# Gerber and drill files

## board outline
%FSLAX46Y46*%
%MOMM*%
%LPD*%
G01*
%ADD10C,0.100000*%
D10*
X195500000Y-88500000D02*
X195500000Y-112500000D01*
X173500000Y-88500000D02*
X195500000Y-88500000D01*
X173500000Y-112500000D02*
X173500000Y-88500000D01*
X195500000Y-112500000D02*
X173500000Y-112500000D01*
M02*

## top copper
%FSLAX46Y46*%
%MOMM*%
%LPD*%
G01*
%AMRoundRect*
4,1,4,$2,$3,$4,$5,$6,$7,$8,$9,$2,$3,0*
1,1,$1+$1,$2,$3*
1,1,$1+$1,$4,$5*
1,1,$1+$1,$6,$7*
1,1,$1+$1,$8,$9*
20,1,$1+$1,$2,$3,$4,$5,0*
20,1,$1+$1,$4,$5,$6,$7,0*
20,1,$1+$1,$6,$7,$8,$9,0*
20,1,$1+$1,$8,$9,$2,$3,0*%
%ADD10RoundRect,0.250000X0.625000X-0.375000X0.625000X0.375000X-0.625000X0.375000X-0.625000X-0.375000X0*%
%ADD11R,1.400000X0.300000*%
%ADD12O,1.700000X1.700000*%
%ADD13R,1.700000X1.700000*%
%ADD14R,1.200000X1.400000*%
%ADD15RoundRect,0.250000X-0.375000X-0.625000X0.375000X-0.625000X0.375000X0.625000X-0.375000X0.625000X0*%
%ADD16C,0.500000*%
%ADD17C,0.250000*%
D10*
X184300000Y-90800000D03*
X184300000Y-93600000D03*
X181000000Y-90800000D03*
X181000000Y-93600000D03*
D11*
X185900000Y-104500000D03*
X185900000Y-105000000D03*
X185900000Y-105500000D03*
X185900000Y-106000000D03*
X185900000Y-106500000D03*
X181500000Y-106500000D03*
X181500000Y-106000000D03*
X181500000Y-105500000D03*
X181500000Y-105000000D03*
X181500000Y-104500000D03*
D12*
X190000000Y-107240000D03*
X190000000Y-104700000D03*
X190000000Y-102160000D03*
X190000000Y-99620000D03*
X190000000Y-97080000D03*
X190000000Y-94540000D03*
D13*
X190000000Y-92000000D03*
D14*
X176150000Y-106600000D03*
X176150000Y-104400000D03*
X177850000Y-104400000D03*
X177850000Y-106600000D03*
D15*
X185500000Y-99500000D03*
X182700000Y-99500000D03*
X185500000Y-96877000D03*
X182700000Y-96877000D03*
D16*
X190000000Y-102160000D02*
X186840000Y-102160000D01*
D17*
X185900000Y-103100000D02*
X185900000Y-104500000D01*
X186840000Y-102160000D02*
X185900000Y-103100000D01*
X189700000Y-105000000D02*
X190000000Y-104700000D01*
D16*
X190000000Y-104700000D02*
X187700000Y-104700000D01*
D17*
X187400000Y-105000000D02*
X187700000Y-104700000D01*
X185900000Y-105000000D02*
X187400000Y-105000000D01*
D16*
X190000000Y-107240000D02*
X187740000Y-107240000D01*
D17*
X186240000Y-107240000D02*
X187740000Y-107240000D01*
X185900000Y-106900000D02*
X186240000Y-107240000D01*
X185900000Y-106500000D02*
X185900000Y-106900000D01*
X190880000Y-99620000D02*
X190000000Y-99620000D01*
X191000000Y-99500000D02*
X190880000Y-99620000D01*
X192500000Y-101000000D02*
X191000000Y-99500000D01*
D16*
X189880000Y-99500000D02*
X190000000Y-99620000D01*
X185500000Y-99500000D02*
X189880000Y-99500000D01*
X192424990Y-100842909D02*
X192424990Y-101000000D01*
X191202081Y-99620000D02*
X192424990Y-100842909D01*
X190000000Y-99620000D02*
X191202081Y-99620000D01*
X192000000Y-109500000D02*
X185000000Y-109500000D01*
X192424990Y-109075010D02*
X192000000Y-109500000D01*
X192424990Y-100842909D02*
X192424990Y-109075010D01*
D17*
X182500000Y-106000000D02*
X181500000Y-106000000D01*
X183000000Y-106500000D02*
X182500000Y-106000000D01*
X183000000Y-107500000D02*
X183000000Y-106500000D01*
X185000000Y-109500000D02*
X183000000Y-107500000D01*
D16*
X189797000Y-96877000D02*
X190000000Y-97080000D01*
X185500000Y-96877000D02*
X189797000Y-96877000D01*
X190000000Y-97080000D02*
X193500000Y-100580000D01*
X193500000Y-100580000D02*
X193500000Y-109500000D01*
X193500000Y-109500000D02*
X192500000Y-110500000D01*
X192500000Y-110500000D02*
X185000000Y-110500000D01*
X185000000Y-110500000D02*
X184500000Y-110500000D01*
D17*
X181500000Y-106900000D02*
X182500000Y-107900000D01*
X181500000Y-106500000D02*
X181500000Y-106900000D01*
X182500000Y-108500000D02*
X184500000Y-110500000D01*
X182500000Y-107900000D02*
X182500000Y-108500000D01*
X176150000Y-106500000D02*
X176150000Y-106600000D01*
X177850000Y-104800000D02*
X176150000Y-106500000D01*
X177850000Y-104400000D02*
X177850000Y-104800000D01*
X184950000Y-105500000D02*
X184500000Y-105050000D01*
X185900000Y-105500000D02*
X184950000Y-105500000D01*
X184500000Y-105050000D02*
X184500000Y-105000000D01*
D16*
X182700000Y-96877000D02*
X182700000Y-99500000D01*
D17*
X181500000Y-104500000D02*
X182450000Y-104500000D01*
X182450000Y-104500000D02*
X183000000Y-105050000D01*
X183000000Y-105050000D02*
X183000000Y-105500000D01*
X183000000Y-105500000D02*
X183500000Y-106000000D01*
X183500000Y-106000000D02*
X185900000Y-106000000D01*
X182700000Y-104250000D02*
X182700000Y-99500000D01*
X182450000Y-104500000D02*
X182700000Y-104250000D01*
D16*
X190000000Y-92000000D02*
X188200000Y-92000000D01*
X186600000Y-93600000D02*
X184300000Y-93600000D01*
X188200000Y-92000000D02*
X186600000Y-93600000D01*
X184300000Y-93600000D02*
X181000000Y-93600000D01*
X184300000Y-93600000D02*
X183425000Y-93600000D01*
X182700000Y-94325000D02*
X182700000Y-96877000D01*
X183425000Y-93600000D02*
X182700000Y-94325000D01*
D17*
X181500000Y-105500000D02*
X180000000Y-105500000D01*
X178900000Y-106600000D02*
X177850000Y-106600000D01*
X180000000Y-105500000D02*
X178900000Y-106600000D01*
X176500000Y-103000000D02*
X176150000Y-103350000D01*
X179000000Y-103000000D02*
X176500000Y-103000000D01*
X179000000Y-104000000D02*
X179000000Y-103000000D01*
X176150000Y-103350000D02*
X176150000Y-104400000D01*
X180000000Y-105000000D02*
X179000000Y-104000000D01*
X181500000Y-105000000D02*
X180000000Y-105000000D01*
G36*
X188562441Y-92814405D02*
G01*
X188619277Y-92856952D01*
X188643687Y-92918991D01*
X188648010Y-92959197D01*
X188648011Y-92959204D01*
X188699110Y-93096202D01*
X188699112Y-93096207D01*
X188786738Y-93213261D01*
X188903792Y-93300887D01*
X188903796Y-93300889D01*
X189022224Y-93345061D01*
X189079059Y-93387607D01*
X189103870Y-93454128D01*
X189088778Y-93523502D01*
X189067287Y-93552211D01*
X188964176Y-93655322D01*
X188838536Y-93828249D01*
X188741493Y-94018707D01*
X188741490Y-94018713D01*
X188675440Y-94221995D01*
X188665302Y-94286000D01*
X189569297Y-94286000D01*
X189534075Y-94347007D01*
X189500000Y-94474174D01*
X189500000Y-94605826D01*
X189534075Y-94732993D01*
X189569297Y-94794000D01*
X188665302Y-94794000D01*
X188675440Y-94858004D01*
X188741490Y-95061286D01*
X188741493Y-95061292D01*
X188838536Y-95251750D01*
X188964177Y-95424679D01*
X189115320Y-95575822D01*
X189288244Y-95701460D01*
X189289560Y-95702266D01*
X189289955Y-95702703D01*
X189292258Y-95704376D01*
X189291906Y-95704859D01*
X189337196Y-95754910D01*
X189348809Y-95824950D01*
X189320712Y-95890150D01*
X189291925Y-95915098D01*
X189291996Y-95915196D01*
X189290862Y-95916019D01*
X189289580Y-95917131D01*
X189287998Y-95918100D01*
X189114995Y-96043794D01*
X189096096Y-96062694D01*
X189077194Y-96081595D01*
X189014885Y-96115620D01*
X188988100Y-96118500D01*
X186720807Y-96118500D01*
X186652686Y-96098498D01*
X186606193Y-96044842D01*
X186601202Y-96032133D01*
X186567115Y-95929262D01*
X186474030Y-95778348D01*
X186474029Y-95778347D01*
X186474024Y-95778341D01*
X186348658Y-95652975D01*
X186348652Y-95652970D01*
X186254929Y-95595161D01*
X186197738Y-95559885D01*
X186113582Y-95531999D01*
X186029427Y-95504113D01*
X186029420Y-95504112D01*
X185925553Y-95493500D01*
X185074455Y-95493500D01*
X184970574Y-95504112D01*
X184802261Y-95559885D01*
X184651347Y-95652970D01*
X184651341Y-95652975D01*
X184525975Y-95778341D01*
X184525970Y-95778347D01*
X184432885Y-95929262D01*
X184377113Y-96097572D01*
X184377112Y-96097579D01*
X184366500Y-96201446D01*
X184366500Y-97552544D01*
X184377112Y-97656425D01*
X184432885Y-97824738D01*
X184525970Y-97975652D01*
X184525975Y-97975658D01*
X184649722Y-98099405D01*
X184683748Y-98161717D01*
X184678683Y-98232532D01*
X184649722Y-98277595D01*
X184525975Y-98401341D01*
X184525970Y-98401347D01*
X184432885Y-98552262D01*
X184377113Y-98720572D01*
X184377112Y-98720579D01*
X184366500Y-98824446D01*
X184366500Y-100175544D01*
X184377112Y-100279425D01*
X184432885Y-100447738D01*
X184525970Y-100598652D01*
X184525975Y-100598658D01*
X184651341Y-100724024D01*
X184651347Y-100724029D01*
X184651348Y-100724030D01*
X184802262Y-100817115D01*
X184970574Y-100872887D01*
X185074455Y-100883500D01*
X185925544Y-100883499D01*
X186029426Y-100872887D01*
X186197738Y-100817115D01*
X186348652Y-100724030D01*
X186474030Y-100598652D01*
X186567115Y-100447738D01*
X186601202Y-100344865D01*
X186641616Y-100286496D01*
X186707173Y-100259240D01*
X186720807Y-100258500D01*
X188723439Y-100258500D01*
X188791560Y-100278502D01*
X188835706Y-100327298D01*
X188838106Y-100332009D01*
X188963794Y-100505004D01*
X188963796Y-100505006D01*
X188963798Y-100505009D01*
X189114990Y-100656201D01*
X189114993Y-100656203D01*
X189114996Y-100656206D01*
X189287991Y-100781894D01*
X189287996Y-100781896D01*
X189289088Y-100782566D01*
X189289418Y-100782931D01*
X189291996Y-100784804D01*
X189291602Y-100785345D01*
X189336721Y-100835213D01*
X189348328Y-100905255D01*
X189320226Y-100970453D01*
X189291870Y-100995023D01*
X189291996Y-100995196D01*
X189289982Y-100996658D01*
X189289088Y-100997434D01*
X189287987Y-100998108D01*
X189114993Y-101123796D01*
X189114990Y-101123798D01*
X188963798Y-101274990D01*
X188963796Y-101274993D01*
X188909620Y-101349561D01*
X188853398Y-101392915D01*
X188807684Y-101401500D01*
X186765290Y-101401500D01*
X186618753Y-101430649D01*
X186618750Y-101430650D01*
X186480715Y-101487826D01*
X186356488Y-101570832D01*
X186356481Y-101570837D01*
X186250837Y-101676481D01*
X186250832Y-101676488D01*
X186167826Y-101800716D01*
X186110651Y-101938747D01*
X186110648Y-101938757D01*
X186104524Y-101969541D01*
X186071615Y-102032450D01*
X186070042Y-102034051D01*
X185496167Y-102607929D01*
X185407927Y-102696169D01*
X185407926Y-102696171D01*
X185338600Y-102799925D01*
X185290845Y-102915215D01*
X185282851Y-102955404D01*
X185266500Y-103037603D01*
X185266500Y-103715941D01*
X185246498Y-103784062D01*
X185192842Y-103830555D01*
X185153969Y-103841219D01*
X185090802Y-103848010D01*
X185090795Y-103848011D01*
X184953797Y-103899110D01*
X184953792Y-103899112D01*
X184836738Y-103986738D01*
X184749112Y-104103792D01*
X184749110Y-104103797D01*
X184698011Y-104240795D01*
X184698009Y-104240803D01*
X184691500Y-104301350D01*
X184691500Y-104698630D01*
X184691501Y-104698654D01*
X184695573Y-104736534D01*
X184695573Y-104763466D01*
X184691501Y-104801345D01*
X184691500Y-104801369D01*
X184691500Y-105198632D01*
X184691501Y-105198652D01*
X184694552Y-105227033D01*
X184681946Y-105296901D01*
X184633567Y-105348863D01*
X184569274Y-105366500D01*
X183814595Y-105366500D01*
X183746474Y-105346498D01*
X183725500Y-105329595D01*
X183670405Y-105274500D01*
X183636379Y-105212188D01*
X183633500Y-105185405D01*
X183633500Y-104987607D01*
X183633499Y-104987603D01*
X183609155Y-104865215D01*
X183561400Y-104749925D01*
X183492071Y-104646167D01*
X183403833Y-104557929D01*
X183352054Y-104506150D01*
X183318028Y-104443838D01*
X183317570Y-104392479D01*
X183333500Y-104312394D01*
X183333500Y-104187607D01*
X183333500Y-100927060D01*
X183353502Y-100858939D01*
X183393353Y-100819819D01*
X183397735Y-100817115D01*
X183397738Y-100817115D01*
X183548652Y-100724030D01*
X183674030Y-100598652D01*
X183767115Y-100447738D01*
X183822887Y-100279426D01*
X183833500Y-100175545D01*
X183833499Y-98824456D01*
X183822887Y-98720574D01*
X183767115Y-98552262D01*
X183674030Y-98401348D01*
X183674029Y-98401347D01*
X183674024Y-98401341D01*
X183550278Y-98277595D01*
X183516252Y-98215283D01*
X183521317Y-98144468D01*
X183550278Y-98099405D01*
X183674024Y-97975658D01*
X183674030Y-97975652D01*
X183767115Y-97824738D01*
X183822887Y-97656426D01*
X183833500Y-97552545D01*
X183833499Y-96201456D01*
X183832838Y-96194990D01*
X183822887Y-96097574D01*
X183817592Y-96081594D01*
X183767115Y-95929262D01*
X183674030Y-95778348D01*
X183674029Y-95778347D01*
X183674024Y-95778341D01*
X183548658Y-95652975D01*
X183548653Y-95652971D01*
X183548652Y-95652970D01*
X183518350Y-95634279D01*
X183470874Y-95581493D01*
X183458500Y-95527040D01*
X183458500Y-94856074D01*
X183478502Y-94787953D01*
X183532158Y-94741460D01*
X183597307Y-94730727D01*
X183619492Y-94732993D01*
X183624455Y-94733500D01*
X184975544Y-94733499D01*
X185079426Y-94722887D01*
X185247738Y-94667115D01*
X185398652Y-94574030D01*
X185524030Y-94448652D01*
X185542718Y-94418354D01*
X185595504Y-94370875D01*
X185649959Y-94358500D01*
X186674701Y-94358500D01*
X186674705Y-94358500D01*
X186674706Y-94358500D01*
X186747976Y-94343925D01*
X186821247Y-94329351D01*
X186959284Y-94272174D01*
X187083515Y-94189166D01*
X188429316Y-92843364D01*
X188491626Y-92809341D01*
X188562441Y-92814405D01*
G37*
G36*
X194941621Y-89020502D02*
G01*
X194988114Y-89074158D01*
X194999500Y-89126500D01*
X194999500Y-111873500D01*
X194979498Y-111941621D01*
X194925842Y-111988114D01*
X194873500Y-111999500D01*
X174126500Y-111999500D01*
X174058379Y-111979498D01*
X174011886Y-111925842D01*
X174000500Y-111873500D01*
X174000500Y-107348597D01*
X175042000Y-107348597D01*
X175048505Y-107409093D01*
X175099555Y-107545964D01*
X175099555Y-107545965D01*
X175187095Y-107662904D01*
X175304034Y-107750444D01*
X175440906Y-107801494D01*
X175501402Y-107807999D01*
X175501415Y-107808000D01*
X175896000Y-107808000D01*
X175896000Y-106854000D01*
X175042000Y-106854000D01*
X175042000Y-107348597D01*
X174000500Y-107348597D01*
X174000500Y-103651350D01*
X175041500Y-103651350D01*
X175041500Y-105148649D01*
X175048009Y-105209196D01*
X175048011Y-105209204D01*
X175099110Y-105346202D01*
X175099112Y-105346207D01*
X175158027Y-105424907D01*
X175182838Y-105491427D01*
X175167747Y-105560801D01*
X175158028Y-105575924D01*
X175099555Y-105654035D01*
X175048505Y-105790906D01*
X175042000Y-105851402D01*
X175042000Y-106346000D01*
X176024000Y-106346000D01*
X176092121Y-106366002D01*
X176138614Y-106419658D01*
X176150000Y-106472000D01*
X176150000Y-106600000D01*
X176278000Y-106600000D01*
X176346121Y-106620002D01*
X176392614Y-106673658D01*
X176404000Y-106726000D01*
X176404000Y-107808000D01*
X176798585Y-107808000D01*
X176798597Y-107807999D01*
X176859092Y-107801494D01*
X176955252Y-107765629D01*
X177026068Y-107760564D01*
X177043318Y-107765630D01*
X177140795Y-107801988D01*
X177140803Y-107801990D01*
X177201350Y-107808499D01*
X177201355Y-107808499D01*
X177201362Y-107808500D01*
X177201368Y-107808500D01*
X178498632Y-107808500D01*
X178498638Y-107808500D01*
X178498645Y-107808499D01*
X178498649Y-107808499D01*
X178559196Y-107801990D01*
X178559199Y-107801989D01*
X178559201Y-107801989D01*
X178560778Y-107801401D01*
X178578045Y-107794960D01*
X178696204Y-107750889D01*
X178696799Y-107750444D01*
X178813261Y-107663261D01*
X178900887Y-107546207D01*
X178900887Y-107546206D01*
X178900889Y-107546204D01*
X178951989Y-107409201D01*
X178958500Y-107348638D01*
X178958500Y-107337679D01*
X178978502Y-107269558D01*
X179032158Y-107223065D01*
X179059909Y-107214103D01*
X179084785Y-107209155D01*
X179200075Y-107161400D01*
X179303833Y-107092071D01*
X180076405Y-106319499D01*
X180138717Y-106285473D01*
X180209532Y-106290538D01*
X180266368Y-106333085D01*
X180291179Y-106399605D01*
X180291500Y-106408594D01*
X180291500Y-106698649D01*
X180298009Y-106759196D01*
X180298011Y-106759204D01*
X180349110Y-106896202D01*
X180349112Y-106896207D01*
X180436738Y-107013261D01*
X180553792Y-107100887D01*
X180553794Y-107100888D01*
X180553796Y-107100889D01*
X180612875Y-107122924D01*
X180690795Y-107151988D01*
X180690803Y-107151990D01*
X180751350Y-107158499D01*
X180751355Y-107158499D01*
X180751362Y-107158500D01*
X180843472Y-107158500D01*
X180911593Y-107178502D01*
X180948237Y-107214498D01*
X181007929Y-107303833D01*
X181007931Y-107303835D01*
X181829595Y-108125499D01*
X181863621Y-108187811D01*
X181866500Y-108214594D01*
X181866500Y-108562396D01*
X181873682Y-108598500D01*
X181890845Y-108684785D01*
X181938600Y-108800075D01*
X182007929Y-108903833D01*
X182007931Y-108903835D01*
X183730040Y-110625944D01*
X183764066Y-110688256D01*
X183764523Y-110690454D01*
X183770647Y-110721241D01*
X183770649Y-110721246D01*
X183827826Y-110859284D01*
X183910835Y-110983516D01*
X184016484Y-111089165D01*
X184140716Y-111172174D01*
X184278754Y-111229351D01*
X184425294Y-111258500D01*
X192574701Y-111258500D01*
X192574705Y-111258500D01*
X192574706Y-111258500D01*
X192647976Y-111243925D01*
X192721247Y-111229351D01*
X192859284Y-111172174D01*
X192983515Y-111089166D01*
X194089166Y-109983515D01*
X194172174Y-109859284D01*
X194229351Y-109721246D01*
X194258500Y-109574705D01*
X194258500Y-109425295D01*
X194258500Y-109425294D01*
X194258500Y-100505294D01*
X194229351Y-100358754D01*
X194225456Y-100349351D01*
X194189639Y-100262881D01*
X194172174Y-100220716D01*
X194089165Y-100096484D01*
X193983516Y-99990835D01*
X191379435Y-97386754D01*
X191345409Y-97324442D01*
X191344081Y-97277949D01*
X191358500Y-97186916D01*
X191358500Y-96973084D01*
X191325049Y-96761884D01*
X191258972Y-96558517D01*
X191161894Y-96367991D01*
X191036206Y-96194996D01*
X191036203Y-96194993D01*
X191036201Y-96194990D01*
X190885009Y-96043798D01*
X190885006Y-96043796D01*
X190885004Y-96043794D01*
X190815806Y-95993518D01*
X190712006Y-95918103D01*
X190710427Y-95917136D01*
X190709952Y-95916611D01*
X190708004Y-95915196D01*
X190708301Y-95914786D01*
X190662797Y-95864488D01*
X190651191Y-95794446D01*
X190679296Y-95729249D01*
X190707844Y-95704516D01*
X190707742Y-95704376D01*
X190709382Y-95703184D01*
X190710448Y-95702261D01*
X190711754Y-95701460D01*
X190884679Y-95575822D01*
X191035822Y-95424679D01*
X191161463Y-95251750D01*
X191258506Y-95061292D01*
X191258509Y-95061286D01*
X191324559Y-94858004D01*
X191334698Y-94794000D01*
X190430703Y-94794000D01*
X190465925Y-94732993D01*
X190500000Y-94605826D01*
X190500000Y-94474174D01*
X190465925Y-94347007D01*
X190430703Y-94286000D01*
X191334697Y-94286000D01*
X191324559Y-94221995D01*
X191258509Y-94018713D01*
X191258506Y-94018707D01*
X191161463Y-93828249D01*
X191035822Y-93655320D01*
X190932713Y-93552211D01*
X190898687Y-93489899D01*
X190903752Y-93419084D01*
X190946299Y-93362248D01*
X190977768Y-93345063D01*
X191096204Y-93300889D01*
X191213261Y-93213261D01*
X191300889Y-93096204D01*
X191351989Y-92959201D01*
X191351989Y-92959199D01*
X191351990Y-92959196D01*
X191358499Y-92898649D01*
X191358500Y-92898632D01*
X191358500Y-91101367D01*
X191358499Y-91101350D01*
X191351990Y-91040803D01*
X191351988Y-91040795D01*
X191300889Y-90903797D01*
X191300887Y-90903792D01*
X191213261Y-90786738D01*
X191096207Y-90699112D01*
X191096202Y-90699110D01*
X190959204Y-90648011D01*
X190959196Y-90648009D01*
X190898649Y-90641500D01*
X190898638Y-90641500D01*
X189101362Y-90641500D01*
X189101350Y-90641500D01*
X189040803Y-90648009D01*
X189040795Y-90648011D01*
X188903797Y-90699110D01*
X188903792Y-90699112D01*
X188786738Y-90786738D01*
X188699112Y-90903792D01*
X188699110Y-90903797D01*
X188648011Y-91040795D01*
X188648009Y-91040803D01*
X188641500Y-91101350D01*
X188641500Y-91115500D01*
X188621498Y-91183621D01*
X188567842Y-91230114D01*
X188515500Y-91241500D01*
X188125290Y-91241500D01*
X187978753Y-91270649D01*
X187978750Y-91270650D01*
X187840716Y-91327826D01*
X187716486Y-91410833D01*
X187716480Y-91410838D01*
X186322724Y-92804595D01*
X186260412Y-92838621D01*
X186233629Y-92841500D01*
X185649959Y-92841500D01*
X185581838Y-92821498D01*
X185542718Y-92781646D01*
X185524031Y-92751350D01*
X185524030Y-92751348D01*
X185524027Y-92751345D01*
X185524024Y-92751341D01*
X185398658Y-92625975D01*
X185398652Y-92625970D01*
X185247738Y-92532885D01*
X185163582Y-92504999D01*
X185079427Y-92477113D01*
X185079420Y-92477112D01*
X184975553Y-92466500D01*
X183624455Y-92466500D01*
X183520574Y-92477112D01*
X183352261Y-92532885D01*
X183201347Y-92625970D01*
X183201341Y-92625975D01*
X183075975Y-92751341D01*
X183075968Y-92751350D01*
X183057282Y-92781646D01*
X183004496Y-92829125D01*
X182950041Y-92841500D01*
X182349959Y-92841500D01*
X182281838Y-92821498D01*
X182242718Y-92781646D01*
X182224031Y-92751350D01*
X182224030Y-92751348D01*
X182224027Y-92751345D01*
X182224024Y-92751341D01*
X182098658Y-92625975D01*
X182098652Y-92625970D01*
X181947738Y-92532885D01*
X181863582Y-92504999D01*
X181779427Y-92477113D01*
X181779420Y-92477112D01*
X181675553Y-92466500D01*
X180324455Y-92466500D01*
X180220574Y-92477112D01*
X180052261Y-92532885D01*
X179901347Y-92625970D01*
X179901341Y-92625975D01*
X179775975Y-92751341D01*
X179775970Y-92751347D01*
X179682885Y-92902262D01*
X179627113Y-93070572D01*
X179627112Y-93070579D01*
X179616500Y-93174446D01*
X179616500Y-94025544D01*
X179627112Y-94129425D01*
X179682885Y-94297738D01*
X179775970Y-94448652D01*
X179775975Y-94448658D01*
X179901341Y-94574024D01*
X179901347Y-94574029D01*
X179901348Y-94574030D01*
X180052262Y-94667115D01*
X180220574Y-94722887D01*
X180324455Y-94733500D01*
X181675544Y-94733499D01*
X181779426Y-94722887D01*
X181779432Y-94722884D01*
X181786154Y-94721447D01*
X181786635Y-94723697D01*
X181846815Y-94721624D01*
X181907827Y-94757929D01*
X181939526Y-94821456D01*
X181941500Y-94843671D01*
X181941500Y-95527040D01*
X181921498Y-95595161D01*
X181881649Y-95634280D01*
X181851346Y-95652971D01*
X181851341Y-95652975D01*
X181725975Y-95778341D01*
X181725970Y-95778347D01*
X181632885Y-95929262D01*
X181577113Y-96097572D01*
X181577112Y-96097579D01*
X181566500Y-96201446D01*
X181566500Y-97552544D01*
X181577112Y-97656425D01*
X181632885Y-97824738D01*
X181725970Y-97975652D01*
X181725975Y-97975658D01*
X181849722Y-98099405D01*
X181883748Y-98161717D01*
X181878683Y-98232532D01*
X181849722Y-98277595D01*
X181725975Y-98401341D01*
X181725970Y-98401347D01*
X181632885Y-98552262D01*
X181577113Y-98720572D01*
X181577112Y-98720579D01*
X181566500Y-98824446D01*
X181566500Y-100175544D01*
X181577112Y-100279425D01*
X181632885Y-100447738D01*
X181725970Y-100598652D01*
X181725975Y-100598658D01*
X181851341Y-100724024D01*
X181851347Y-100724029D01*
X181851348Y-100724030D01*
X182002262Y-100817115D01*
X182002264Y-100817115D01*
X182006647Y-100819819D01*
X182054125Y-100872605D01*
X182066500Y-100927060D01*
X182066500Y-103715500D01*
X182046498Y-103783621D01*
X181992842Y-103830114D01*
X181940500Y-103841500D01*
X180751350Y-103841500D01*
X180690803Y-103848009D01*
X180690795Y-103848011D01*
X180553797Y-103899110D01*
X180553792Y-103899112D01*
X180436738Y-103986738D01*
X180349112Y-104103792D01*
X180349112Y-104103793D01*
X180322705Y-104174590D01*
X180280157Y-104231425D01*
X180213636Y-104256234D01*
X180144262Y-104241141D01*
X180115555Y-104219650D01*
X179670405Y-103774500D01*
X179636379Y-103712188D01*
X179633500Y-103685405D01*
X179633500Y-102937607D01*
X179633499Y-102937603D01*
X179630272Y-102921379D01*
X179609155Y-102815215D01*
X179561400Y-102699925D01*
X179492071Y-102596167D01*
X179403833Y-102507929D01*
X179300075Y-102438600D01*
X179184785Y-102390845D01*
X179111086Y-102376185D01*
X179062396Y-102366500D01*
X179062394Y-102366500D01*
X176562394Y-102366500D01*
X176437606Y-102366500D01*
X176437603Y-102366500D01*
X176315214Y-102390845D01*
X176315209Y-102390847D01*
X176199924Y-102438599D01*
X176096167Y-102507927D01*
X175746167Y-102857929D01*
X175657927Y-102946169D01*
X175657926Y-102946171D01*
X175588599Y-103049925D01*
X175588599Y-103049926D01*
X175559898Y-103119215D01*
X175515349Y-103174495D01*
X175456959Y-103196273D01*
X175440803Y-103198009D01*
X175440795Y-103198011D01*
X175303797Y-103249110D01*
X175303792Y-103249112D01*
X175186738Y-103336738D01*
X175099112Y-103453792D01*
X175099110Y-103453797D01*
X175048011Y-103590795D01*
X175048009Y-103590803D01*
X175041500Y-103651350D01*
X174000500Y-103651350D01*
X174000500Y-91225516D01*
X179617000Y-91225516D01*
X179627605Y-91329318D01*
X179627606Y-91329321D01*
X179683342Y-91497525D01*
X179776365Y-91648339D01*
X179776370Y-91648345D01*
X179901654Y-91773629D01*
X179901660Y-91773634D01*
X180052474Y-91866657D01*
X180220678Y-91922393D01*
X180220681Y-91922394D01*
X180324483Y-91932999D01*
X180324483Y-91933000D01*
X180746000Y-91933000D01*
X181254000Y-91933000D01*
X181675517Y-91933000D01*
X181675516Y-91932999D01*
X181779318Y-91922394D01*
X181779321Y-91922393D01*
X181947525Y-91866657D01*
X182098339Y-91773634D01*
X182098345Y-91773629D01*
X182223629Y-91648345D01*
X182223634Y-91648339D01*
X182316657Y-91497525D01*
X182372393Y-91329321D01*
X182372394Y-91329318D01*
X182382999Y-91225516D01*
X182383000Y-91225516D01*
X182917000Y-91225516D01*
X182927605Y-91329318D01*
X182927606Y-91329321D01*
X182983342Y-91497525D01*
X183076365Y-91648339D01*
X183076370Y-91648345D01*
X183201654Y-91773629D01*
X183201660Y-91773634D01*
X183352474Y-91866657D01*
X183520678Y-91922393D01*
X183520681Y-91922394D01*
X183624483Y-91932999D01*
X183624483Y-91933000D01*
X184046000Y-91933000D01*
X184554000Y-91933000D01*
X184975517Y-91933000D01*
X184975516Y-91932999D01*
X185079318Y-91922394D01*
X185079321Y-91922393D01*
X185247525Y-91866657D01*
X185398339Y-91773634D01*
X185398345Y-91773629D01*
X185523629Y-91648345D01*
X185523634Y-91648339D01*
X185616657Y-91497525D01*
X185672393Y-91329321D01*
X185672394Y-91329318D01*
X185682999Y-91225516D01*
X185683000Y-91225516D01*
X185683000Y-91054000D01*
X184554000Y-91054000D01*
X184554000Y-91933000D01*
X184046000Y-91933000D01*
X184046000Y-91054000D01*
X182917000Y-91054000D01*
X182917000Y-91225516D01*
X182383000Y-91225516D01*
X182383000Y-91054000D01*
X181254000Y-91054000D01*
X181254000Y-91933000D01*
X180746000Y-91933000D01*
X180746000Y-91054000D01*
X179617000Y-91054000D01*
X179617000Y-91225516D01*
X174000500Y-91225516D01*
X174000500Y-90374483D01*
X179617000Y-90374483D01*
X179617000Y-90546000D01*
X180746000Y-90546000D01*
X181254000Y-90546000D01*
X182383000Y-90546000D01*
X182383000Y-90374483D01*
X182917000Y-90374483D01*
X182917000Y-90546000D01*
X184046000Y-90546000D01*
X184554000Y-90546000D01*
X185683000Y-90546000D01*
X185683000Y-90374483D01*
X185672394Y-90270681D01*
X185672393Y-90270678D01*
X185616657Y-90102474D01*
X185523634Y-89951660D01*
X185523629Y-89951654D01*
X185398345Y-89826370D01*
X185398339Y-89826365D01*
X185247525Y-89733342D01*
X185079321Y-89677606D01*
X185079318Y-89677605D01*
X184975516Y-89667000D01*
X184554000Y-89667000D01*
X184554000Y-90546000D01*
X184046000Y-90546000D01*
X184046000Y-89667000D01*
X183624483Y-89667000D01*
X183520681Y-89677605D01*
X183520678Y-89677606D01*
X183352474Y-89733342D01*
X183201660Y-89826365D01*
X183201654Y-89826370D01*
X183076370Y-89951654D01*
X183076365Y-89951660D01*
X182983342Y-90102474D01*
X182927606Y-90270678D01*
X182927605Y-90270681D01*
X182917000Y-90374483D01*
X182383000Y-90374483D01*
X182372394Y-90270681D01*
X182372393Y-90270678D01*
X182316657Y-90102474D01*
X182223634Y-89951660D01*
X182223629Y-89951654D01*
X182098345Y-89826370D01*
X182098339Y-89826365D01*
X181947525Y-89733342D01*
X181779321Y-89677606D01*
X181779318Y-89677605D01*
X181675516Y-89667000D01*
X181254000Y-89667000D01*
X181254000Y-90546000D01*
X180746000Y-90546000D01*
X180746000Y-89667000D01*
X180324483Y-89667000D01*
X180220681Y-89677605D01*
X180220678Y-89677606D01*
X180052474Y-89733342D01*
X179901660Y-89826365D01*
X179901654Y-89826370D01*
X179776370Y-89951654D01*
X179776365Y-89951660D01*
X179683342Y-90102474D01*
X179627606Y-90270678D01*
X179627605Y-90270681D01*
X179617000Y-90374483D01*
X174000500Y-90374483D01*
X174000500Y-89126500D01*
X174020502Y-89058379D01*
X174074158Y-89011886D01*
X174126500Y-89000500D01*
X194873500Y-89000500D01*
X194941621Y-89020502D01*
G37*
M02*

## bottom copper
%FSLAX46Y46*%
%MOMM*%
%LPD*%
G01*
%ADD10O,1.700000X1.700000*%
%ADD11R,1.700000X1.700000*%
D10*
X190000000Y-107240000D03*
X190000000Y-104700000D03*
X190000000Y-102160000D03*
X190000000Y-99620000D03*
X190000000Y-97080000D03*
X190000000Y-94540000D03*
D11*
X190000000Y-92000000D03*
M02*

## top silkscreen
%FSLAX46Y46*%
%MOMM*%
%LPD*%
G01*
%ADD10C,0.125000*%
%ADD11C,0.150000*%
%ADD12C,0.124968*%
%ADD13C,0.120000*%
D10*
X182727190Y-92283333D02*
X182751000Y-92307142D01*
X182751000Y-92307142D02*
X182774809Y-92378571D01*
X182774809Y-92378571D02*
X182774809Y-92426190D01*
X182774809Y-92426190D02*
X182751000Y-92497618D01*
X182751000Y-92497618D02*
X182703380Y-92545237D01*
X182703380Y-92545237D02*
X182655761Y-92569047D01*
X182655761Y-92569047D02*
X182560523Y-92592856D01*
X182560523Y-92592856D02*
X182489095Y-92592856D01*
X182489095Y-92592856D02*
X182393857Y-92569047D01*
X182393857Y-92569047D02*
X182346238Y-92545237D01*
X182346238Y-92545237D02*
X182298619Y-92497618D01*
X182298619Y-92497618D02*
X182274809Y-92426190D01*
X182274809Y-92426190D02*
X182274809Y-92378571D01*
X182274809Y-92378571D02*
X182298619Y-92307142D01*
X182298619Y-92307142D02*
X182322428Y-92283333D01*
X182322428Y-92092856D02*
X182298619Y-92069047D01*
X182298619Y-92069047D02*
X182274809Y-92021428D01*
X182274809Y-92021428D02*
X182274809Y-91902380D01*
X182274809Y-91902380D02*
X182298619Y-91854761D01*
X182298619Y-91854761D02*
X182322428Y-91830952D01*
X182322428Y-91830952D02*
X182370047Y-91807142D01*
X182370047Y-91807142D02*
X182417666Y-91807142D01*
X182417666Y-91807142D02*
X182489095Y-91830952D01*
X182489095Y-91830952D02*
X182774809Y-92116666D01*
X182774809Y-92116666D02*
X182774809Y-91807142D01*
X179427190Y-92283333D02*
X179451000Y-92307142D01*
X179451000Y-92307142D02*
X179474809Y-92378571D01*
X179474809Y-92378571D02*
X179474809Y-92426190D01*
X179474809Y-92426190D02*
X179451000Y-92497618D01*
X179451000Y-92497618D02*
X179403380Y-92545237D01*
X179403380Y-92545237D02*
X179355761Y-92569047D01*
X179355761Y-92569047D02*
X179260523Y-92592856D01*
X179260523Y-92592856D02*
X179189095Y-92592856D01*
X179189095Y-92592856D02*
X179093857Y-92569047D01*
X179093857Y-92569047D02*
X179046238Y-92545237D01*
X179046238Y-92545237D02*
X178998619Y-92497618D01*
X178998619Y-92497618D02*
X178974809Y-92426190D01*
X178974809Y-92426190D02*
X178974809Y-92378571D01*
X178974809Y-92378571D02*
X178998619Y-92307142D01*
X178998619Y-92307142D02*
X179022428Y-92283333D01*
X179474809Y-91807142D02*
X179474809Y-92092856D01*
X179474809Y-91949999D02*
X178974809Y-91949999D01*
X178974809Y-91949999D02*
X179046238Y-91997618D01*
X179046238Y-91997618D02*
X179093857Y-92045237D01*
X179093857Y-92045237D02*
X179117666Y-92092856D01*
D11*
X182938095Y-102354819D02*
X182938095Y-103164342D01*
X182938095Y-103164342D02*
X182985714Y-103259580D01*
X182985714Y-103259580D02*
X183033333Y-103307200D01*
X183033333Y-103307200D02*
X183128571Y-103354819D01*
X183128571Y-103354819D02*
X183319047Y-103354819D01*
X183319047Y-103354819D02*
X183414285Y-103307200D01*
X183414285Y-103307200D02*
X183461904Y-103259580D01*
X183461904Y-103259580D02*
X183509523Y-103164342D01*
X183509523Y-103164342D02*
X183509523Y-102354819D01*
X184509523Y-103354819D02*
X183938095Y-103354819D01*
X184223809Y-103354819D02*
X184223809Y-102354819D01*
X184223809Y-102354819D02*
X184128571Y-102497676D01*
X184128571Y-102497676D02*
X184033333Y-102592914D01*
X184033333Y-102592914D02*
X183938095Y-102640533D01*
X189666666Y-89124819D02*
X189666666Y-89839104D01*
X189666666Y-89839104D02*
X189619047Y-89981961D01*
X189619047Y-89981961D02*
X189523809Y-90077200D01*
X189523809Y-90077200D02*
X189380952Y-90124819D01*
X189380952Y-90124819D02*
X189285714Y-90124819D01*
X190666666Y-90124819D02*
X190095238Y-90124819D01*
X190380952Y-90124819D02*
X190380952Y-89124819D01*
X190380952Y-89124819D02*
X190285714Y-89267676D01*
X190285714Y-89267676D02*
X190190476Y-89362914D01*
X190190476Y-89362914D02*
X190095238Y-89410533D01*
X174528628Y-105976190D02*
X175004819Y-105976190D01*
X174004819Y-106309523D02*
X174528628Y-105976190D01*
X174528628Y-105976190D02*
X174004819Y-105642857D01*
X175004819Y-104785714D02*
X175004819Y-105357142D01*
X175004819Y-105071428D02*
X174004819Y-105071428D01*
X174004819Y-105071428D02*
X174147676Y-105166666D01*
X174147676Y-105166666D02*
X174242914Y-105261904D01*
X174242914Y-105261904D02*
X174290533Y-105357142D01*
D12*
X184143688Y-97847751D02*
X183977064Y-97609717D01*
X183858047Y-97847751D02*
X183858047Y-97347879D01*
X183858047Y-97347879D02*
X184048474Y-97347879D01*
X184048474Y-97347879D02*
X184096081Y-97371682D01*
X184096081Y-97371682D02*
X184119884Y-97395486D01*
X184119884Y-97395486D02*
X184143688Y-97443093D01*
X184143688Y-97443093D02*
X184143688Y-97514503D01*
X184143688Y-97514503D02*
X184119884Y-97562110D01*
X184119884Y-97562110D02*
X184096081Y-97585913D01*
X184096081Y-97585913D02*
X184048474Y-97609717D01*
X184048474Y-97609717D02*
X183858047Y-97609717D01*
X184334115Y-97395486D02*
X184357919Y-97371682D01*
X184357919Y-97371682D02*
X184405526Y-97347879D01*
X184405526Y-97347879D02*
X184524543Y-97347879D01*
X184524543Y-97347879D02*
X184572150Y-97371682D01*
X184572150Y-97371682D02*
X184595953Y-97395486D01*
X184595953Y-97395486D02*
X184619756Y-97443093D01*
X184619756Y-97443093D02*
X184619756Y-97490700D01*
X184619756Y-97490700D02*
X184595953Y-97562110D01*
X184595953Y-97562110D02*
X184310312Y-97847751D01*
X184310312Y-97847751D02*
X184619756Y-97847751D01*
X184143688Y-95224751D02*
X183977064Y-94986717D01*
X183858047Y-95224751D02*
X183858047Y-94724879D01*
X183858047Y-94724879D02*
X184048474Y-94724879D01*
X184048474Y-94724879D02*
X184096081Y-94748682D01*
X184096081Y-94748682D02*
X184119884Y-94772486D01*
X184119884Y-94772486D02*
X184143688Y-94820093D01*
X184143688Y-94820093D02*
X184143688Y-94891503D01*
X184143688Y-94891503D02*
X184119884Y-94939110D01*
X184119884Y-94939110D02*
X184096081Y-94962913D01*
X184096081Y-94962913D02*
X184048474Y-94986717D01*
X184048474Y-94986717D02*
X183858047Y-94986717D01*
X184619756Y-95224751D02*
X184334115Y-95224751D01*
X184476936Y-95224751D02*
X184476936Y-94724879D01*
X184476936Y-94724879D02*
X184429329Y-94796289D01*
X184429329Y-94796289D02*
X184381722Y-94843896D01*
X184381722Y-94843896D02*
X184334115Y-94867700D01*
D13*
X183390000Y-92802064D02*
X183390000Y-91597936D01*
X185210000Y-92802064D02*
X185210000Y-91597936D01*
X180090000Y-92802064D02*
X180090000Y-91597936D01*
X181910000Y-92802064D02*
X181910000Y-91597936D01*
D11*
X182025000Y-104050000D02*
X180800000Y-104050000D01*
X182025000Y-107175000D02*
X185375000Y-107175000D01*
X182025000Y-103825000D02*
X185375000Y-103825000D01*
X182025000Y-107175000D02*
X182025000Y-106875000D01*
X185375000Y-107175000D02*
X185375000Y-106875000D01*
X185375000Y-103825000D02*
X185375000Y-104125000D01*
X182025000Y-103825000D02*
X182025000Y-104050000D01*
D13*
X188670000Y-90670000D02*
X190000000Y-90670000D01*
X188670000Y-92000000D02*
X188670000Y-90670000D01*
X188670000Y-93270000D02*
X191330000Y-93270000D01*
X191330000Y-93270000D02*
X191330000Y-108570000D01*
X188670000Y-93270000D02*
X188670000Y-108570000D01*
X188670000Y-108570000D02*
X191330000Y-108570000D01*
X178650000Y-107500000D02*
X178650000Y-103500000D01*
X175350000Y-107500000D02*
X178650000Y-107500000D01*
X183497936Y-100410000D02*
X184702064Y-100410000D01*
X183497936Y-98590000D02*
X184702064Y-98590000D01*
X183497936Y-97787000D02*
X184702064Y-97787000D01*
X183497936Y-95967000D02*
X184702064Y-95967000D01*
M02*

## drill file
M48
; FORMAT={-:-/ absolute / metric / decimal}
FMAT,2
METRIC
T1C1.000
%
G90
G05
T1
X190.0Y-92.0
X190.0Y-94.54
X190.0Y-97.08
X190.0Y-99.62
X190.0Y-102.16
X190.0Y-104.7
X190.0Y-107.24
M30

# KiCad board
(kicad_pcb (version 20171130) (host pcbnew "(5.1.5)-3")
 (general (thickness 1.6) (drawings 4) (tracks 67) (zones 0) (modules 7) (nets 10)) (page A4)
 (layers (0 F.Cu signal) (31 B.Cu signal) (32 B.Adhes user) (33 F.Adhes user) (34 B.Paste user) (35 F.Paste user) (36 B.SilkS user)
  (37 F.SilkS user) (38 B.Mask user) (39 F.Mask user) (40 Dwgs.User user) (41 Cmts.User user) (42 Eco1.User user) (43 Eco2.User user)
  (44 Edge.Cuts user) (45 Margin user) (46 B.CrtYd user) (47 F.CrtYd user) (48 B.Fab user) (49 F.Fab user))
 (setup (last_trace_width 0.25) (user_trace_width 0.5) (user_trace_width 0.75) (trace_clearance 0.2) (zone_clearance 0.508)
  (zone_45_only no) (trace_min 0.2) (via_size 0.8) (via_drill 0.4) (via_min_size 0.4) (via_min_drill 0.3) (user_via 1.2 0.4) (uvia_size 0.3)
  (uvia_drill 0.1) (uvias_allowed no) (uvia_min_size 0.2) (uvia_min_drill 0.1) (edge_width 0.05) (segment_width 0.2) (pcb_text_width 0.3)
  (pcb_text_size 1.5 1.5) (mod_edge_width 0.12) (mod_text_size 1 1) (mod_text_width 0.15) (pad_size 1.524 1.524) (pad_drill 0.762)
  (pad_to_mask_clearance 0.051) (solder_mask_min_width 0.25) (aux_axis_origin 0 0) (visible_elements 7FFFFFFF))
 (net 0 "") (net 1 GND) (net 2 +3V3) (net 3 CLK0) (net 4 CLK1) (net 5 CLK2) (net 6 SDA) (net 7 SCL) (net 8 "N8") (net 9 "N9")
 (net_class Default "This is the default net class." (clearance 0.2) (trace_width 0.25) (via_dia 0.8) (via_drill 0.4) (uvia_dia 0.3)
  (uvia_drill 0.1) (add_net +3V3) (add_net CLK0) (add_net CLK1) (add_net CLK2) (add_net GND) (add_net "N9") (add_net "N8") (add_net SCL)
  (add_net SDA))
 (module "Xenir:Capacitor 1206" (layer F.Cu) (at 182.05 92.2 90)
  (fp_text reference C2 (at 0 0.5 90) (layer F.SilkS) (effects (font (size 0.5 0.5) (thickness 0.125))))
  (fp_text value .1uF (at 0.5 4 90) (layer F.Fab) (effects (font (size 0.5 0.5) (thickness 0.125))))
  (fp_line (start -0.602064 1.34) (end 0.602064 1.34) (layer F.SilkS) (width 0.12))
  (fp_line (start -0.602064 3.16) (end 0.602064 3.16) (layer F.SilkS) (width 0.12))
  (pad 2 smd roundrect (at 1.4 2.25 90) (size 1.25 1.75) (layers F.Cu F.Paste F.Mask) (roundrect_rratio 0.2) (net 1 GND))
  (pad 1 smd roundrect (at -1.4 2.25 90) (size 1.25 1.75) (layers F.Cu F.Paste F.Mask) (roundrect_rratio 0.2) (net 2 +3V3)))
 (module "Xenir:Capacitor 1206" (layer F.Cu) (at 178.75 92.2 90)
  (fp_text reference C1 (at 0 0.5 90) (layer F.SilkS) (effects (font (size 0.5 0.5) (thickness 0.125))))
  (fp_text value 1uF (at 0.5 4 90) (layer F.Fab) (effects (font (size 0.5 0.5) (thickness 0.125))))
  (fp_line (start -0.602064 1.34) (end 0.602064 1.34) (layer F.SilkS) (width 0.12))
  (fp_line (start -0.602064 3.16) (end 0.602064 3.16) (layer F.SilkS) (width 0.12))
  (pad 2 smd roundrect (at 1.4 2.25 90) (size 1.25 1.75) (layers F.Cu F.Paste F.Mask) (roundrect_rratio 0.2) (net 1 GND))
  (pad 1 smd roundrect (at -1.4 2.25 90) (size 1.25 1.75) (layers F.Cu F.Paste F.Mask) (roundrect_rratio 0.2) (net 2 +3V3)))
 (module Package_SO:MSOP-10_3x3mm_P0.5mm (layer F.Cu) (at 183.7 105.5)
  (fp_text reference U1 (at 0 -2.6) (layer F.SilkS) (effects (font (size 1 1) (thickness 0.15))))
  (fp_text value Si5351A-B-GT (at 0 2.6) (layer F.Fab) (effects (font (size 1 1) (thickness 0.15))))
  (fp_line (start -1.675 -1.45) (end -2.9 -1.45) (layer F.SilkS) (width 0.15))
  (fp_line (start -1.675 1.675) (end 1.675 1.675) (layer F.SilkS) (width 0.15))
  (fp_line (start -1.675 -1.675) (end 1.675 -1.675) (layer F.SilkS) (width 0.15))
  (fp_line (start -1.675 1.675) (end -1.675 1.375) (layer F.SilkS) (width 0.15))
  (fp_line (start 1.675 1.675) (end 1.675 1.375) (layer F.SilkS) (width 0.15))
  (fp_line (start 1.675 -1.675) (end 1.675 -1.375) (layer F.SilkS) (width 0.15))
  (fp_line (start -1.675 -1.675) (end -1.675 -1.45) (layer F.SilkS) (width 0.15))
  (pad 10 smd rect (at 2.2 -1) (size 1.4 0.3) (layers F.Cu F.Paste F.Mask) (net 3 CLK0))
  (pad 9 smd rect (at 2.2 -0.5) (size 1.4 0.3) (layers F.Cu F.Paste F.Mask) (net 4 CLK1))
  (pad 8 smd rect (at 2.2 0) (size 1.4 0.3) (layers F.Cu F.Paste F.Mask) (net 1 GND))
  (pad 7 smd rect (at 2.2 0.5) (size 1.4 0.3) (layers F.Cu F.Paste F.Mask) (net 2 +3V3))
  (pad 6 smd rect (at 2.2 1) (size 1.4 0.3) (layers F.Cu F.Paste F.Mask) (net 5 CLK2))
  (pad 5 smd rect (at -2.2 1) (size 1.4 0.3) (layers F.Cu F.Paste F.Mask) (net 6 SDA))
  (pad 4 smd rect (at -2.2 0.5) (size 1.4 0.3) (layers F.Cu F.Paste F.Mask) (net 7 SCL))
  (pad 3 smd rect (at -2.2 0) (size 1.4 0.3) (layers F.Cu F.Paste F.Mask) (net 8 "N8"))
  (pad 2 smd rect (at -2.2 -0.5) (size 1.4 0.3) (layers F.Cu F.Paste F.Mask) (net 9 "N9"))
  (pad 1 smd rect (at -2.2 -1) (size 1.4 0.3) (layers F.Cu F.Paste F.Mask) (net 2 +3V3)))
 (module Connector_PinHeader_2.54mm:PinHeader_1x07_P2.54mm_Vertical (layer F.Cu) (at 190 92)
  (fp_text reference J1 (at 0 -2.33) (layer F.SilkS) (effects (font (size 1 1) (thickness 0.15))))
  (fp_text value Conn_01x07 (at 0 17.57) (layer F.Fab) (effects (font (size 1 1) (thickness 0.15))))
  (fp_line (start -1.33 -1.33) (end 0 -1.33) (layer F.SilkS) (width 0.12))
  (fp_line (start -1.33 0) (end -1.33 -1.33) (layer F.SilkS) (width 0.12))
  (fp_line (start -1.33 1.27) (end 1.33 1.27) (layer F.SilkS) (width 0.12))
  (fp_line (start 1.33 1.27) (end 1.33 16.57) (layer F.SilkS) (width 0.12))
  (fp_line (start -1.33 1.27) (end -1.33 16.57) (layer F.SilkS) (width 0.12))
  (fp_line (start -1.33 16.57) (end 1.33 16.57) (layer F.SilkS) (width 0.12))
  (pad 7 thru_hole oval (at 0 15.24) (size 1.7 1.7) (drill 1) (layers *.Cu *.Mask) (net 5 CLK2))
  (pad 6 thru_hole oval (at 0 12.7) (size 1.7 1.7) (drill 1) (layers *.Cu *.Mask) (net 4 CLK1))
  (pad 5 thru_hole oval (at 0 10.16) (size 1.7 1.7) (drill 1) (layers *.Cu *.Mask) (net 3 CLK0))
  (pad 4 thru_hole oval (at 0 7.62) (size 1.7 1.7) (drill 1) (layers *.Cu *.Mask) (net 7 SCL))
  (pad 3 thru_hole oval (at 0 5.08) (size 1.7 1.7) (drill 1) (layers *.Cu *.Mask) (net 6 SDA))
  (pad 2 thru_hole oval (at 0 2.54) (size 1.7 1.7) (drill 1) (layers *.Cu *.Mask) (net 1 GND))
  (pad 1 thru_hole rect (at 0 0) (size 1.7 1.7) (drill 1) (layers *.Cu *.Mask) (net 2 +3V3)))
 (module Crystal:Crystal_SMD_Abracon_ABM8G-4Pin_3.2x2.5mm (layer F.Cu) (at 177 105.5 90)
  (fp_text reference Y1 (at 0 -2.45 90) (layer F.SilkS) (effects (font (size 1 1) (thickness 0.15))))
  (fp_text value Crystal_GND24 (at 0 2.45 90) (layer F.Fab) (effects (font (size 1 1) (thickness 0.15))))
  (fp_line (start -2 1.65) (end 2 1.65) (layer F.SilkS) (width 0.12))
  (fp_line (start -2 -1.65) (end -2 1.65) (layer F.SilkS) (width 0.12))
  (pad 4 smd rect (at -1.1 -0.85 90) (size 1.4 1.2) (layers F.Cu F.Paste F.Mask) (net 1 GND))
  (pad 3 smd rect (at 1.1 -0.85 90) (size 1.4 1.2) (layers F.Cu F.Paste F.Mask) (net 9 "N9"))
  (pad 2 smd rect (at 1.1 0.85 90) (size 1.4 1.2) (layers F.Cu F.Paste F.Mask) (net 1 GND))
  (pad 1 smd rect (at -1.1 0.85 90) (size 1.4 1.2) (layers F.Cu F.Paste F.Mask) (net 8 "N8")))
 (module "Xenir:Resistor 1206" (layer F.Cu) (at 184.227 97.123)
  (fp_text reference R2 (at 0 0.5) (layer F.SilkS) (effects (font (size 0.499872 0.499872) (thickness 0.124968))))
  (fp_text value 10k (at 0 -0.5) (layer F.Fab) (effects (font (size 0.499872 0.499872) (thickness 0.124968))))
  (fp_line (start -0.729064 3.287) (end 0.475064 3.287) (layer F.SilkS) (width 0.12))
  (fp_line (start -0.729064 1.467) (end 0.475064 1.467) (layer F.SilkS) (width 0.12))
  (pad 2 smd roundrect (at 1.273 2.377) (size 1.25 1.75) (layers F.Cu F.Paste F.Mask) (roundrect_rratio 0.2) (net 7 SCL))
  (pad 1 smd roundrect (at -1.527 2.377) (size 1.25 1.75) (layers F.Cu F.Paste F.Mask) (roundrect_rratio 0.2) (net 2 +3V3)))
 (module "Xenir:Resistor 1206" (layer F.Cu) (at 184.227 94.5)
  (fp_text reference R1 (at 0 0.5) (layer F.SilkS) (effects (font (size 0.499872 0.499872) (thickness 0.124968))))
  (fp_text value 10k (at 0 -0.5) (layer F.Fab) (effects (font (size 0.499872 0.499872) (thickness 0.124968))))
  (fp_line (start -0.729064 3.287) (end 0.475064 3.287) (layer F.SilkS) (width 0.12))
  (fp_line (start -0.729064 1.467) (end 0.475064 1.467) (layer F.SilkS) (width 0.12))
  (pad 2 smd roundrect (at 1.273 2.377) (size 1.25 1.75) (layers F.Cu F.Paste F.Mask) (roundrect_rratio 0.2) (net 6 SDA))
  (pad 1 smd roundrect (at -1.527 2.377) (size 1.25 1.75) (layers F.Cu F.Paste F.Mask) (roundrect_rratio 0.2) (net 2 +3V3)))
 (gr_line (start 195.5 88.5) (end 195.5 112.5) (layer Edge.Cuts) (width 0.1))
 (gr_line (start 173.5 88.5) (end 195.5 88.5) (layer Edge.Cuts) (width 0.1))
 (gr_line (start 173.5 112.5) (end 173.5 88.5) (layer Edge.Cuts) (width 0.1))
 (gr_line (start 195.5 112.5) (end 173.5 112.5) (layer Edge.Cuts) (width 0.1))
 (segment (start 190 102.16) (end 186.84 102.16) (width 0.5) (layer F.Cu) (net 3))
 (segment (start 185.9 103.1) (end 185.9 104.5) (width 0.25) (layer F.Cu) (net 3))
 (segment (start 186.84 102.16) (end 185.9 103.1) (width 0.25) (layer F.Cu) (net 3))
 (segment (start 189.7 105) (end 190 104.7) (width 0.25) (layer F.Cu) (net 4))
 (segment (start 190 104.7) (end 187.7 104.7) (width 0.5) (layer F.Cu) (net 4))
 (segment (start 187.4 105) (end 187.7 104.7) (width 0.25) (layer F.Cu) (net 4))
 (segment (start 185.9 105) (end 187.4 105) (width 0.25) (layer F.Cu) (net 4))
 (segment (start 190 107.24) (end 187.74 107.24) (width 0.5) (layer F.Cu) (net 5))
 (segment (start 186.24 107.24) (end 187.74 107.24) (width 0.25) (layer F.Cu) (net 5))
 (segment (start 185.9 106.9) (end 186.24 107.24) (width 0.25) (layer F.Cu) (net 5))
 (segment (start 185.9 106.5) (end 185.9 106.9) (width 0.25) (layer F.Cu) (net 5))
 (segment (start 190.88 99.62) (end 190 99.62) (width 0.25) (layer F.Cu) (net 7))
 (segment (start 191 99.5) (end 190.88 99.62) (width 0.25) (layer F.Cu) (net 7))
 (segment (start 192.5 101) (end 191 99.5) (width 0.25) (layer F.Cu) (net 7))
 (segment (start 189.88 99.5) (end 190 99.62) (width 0.5) (layer F.Cu) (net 7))
 (segment (start 185.5 99.5) (end 189.88 99.5) (width 0.5) (layer F.Cu) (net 7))
 (segment (start 192.42499 100.842909) (end 192.42499 101) (width 0.5) (layer F.Cu) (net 7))
 (segment (start 191.202081 99.62) (end 192.42499 100.842909) (width 0.5) (layer F.Cu) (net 7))
 (segment (start 190 99.62) (end 191.202081 99.62) (width 0.5) (layer F.Cu) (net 7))
 (segment (start 192 109.5) (end 185 109.5) (width 0.5) (layer F.Cu) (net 7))
 (segment (start 192.42499 109.07501) (end 192 109.5) (width 0.5) (layer F.Cu) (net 7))
 (segment (start 192.42499 100.842909) (end 192.42499 109.07501) (width 0.5) (layer F.Cu) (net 7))
 (segment (start 182.5 106) (end 181.5 106) (width 0.25) (layer F.Cu) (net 7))
 (segment (start 183 106.5) (end 182.5 106) (width 0.25) (layer F.Cu) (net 7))
 (segment (start 183 107.5) (end 183 106.5) (width 0.25) (layer F.Cu) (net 7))
 (segment (start 185 109.5) (end 183 107.5) (width 0.25) (layer F.Cu) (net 7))
 (segment (start 189.797 96.877) (end 190 97.08) (width 0.5) (layer F.Cu) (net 6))
 (segment (start 185.5 96.877) (end 189.797 96.877) (width 0.5) (layer F.Cu) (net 6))
 (segment (start 190 97.08) (end 193.5 100.58) (width 0.5) (layer F.Cu) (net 6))
 (segment (start 193.5 100.58) (end 193.5 109.5) (width 0.5) (layer F.Cu) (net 6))
 (segment (start 193.5 109.5) (end 192.5 110.5) (width 0.5) (layer F.Cu) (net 6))
 (segment (start 192.5 110.5) (end 185 110.5) (width 0.5) (layer F.Cu) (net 6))
 (segment (start 185 110.5) (end 184.5 110.5) (width 0.5) (layer F.Cu) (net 6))
 (segment (start 181.5 106.9) (end 182.5 107.9) (width 0.25) (layer F.Cu) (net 6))
 (segment (start 181.5 106.5) (end 181.5 106.9) (width 0.25) (layer F.Cu) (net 6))
 (segment (start 182.5 108.5) (end 184.5 110.5) (width 0.25) (layer F.Cu) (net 6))
 (segment (start 182.5 107.9) (end 182.5 108.5) (width 0.25) (layer F.Cu) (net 6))
 (segment (start 176.15 106.5) (end 176.15 106.6) (width 0.25) (layer F.Cu) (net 1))
 (segment (start 177.85 104.8) (end 176.15 106.5) (width 0.25) (layer F.Cu) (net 1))
 (segment (start 177.85 104.4) (end 177.85 104.8) (width 0.25) (layer F.Cu) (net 1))
 (segment (start 184.95 105.5) (end 184.5 105.05) (width 0.25) (layer F.Cu) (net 1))
 (segment (start 185.9 105.5) (end 184.95 105.5) (width 0.25) (layer F.Cu) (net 1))
 (segment (start 184.5 105.05) (end 184.5 105) (width 0.25) (layer F.Cu) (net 1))
 (segment (start 182.7 96.877) (end 182.7 99.5) (width 0.5) (layer F.Cu) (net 2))
 (segment (start 181.5 104.5) (end 182.45 104.5) (width 0.25) (layer F.Cu) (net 2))
 (segment (start 182.45 104.5) (end 183 105.05) (width 0.25) (layer F.Cu) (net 2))
 (segment (start 183 105.05) (end 183 105.5) (width 0.25) (layer F.Cu) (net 2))
 (segment (start 183 105.5) (end 183.5 106) (width 0.25) (layer F.Cu) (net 2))
 (segment (start 183.5 106) (end 185.9 106) (width 0.25) (layer F.Cu) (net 2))
 (segment (start 182.7 104.25) (end 182.7 99.5) (width 0.25) (layer F.Cu) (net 2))
 (segment (start 182.45 104.5) (end 182.7 104.25) (width 0.25) (layer F.Cu) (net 2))
 (segment (start 190 92) (end 188.2 92) (width 0.5) (layer F.Cu) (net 2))
 (segment (start 186.6 93.6) (end 184.3 93.6) (width 0.5) (layer F.Cu) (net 2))
 (segment (start 188.2 92) (end 186.6 93.6) (width 0.5) (layer F.Cu) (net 2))
 (segment (start 184.3 93.6) (end 181 93.6) (width 0.5) (layer F.Cu) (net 2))
 (segment (start 184.3 93.6) (end 183.425 93.6) (width 0.5) (layer F.Cu) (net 2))
 (segment (start 182.7 94.325) (end 182.7 96.877) (width 0.5) (layer F.Cu) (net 2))
 (segment (start 183.425 93.6) (end 182.7 94.325) (width 0.5) (layer F.Cu) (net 2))
 (segment (start 181.5 105.5) (end 180 105.5) (width 0.25) (layer F.Cu) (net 8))
 (segment (start 178.9 106.6) (end 177.85 106.6) (width 0.25) (layer F.Cu) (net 8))
 (segment (start 180 105.5) (end 178.9 106.6) (width 0.25) (layer F.Cu) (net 8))
 (segment (start 176.5 103) (end 176.15 103.35) (width 0.25) (layer F.Cu) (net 9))
 (segment (start 179 103) (end 176.5 103) (width 0.25) (layer F.Cu) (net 9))
 (segment (start 179 104) (end 179 103) (width 0.25) (layer F.Cu) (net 9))
 (segment (start 176.15 103.35) (end 176.15 104.4) (width 0.25) (layer F.Cu) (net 9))
 (segment (start 180 105) (end 179 104) (width 0.25) (layer F.Cu) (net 9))
 (segment (start 181.5 105) (end 180 105) (width 0.25) (layer F.Cu) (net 9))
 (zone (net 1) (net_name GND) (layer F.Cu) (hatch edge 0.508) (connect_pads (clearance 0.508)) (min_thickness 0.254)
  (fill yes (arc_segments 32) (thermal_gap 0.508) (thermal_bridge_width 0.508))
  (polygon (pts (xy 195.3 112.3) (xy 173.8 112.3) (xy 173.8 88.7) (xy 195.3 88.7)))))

